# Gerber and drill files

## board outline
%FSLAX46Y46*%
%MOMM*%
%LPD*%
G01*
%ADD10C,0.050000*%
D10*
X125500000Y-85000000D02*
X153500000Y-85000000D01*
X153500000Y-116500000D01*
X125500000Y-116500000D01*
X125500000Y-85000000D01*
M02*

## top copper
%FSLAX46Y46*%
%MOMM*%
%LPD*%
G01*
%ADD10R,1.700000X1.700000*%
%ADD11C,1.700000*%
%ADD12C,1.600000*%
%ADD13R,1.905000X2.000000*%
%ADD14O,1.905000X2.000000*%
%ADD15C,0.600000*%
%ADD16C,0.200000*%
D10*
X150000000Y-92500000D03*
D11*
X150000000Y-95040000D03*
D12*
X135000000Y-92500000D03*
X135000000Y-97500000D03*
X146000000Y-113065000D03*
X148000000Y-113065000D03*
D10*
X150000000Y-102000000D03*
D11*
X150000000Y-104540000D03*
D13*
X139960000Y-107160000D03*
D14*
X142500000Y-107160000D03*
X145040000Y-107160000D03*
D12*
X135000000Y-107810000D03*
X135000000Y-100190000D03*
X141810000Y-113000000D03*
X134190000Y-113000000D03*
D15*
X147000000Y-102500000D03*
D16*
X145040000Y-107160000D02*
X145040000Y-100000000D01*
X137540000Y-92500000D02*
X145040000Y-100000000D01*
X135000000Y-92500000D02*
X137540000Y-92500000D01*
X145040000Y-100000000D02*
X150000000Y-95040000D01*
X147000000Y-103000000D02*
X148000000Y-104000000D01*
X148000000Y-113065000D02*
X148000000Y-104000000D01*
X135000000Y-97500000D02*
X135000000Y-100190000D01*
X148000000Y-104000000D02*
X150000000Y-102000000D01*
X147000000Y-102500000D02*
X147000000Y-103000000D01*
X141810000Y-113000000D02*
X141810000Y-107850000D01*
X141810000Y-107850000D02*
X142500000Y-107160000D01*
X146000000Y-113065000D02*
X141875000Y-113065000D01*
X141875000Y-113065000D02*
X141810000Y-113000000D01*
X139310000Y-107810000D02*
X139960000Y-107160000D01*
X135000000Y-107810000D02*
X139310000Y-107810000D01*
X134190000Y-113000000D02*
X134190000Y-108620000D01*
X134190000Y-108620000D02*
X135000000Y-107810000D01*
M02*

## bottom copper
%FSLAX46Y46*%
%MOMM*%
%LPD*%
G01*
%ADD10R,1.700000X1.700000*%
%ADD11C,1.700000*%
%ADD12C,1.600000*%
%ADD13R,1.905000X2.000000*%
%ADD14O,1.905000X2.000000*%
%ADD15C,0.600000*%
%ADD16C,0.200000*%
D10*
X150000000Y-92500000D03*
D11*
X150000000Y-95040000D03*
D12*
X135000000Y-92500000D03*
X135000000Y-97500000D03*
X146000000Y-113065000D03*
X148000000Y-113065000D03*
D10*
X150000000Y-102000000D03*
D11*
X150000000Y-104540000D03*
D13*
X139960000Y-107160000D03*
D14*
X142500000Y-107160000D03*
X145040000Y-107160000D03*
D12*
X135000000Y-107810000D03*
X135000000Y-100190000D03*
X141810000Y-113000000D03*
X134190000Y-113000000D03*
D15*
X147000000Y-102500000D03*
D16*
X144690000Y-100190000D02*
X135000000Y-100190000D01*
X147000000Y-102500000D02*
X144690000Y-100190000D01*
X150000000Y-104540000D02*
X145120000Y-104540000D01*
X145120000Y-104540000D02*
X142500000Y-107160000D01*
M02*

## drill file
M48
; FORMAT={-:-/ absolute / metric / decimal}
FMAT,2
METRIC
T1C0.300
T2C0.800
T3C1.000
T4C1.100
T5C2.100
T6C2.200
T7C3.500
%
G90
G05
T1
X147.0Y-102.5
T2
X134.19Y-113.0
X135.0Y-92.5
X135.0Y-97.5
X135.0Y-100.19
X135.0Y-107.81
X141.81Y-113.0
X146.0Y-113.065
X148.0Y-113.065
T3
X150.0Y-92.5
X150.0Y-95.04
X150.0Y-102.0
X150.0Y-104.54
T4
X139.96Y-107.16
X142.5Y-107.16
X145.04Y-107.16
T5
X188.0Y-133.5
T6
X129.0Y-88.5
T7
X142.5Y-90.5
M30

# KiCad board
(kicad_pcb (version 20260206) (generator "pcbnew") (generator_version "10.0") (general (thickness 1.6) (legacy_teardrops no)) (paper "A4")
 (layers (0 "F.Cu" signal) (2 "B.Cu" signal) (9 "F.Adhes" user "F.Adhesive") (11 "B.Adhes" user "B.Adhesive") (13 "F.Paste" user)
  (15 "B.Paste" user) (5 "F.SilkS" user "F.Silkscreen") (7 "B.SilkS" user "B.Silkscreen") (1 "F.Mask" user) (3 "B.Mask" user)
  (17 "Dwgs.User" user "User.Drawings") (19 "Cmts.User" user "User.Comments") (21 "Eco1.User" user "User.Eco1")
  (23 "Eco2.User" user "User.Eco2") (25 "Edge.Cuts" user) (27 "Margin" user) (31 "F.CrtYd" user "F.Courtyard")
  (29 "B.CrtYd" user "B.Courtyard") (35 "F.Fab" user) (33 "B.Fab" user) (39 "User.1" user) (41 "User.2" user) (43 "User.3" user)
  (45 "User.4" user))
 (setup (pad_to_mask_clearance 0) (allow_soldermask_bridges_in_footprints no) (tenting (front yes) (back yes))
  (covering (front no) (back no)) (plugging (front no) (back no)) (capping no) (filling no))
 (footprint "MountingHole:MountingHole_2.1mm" (layer "F.Cu") (at 188 133.5)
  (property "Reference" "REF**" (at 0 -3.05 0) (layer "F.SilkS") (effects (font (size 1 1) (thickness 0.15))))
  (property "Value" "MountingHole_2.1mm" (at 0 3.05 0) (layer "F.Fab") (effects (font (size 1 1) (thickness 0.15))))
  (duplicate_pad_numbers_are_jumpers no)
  (pad "" np_thru_hole circle (at 0 0) (size 2.1 2.1) (drill 2.1) (layers "*.Cu" "*.Mask")))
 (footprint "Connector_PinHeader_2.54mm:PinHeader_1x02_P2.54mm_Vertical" (layer "F.Cu") (at 150 92.5)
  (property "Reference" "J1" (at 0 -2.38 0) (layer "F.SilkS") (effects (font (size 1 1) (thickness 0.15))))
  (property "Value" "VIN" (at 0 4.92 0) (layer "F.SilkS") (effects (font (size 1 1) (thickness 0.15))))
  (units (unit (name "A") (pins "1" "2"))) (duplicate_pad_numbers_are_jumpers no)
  (pad "1" thru_hole rect (at 0 0) (size 1.7 1.7) (drill 1) (layers "*.Cu" "*.Mask") (remove_unused_layers no) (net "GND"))
  (pad "2" thru_hole circle (at 0 2.54) (size 1.7 1.7) (drill 1) (layers "*.Cu" "*.Mask") (remove_unused_layers no) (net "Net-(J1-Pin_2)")))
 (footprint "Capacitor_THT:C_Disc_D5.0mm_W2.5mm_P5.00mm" (layer "F.Cu") (at 135 92.5 -90)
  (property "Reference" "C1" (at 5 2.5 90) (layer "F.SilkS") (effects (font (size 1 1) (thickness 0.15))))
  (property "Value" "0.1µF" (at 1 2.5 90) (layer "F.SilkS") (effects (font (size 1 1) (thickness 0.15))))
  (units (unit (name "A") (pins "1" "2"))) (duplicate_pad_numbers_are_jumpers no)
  (pad "1" thru_hole circle (at 0 0 270) (size 1.6 1.6) (drill 0.8) (layers "*.Cu" "*.Mask") (remove_unused_layers no)
   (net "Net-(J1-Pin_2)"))
  (pad "2" thru_hole circle (at 5 0 270) (size 1.6 1.6) (drill 0.8) (layers "*.Cu" "*.Mask") (remove_unused_layers no) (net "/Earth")))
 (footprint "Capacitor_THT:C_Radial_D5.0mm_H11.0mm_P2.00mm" (layer "F.Cu") (at 146 113.065)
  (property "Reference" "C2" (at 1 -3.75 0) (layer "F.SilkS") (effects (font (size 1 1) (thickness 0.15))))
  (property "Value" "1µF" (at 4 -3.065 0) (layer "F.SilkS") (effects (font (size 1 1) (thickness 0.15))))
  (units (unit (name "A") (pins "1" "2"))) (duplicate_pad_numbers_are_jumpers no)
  (pad "1" thru_hole circle (at 0 0) (size 1.6 1.6) (drill 0.8) (layers "*.Cu" "*.Mask") (remove_unused_layers no) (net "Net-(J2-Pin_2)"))
  (pad "2" thru_hole circle (at 2 0) (size 1.6 1.6) (drill 0.8) (layers "*.Cu" "*.Mask") (remove_unused_layers no) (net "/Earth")))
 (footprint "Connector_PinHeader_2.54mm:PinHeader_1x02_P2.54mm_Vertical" (layer "F.Cu") (at 150 102)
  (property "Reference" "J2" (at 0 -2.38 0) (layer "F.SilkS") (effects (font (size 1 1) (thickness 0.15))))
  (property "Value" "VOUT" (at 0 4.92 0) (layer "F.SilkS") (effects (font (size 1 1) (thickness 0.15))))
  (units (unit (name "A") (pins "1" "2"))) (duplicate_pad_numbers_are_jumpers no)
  (pad "1" thru_hole rect (at 0 0) (size 1.7 1.7) (drill 1) (layers "*.Cu" "*.Mask") (remove_unused_layers no) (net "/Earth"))
  (pad "2" thru_hole circle (at 0 2.54) (size 1.7 1.7) (drill 1) (layers "*.Cu" "*.Mask") (remove_unused_layers no) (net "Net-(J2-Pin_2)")))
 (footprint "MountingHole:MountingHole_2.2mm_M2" (layer "F.Cu") (at 129 88.5)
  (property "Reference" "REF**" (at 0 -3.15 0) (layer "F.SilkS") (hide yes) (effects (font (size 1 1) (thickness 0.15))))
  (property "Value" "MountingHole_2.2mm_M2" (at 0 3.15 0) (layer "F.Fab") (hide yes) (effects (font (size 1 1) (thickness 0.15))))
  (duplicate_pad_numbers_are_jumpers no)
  (pad "" np_thru_hole circle (at 0 0) (size 2.2 2.2) (drill 2.2) (layers "*.Cu" "*.Mask")))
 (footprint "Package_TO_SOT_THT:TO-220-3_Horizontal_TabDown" (layer "F.Cu") (at 139.96 107.16)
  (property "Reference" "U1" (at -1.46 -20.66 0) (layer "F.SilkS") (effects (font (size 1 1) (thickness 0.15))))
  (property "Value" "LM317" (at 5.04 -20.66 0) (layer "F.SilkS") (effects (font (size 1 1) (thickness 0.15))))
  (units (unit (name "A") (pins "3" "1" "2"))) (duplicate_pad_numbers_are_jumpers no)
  (pad "" np_thru_hole circle (at 2.54 -16.66) (size 3.5 3.5) (drill 3.5) (layers "*.Cu" "*.Mask"))
  (pad "1" thru_hole rect (at 0 0) (size 1.905 2) (drill 1.1) (layers "*.Cu" "*.Mask") (remove_unused_layers no) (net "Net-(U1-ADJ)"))
  (pad "2" thru_hole oval (at 2.54 0) (size 1.905 2) (drill 1.1) (layers "*.Cu" "*.Mask") (remove_unused_layers no) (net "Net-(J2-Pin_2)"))
  (pad "3" thru_hole oval (at 5.08 0) (size 1.905 2) (drill 1.1) (layers "*.Cu" "*.Mask") (remove_unused_layers no) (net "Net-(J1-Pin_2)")))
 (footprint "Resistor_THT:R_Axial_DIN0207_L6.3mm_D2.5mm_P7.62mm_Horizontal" (layer "F.Cu") (at 135 107.81 90)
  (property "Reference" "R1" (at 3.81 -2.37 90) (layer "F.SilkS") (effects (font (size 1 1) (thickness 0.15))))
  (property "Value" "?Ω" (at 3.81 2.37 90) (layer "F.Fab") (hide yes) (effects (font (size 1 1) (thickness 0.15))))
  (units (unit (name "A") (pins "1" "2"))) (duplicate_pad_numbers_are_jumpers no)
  (pad "1" thru_hole circle (at 0 0 90) (size 1.6 1.6) (drill 0.8) (layers "*.Cu" "*.Mask") (remove_unused_layers no) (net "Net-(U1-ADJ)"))
  (pad "2" thru_hole circle (at 7.62 0 90) (size 1.6 1.6) (drill 0.8) (layers "*.Cu" "*.Mask") (remove_unused_layers no) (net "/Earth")))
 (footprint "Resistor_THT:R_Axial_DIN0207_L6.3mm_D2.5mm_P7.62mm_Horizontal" (layer "F.Cu") (at 141.81 113 180)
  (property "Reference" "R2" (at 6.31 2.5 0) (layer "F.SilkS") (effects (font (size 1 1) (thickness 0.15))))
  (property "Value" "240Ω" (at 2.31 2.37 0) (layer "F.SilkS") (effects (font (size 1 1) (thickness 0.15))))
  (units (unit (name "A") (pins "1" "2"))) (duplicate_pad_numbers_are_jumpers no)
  (pad "1" thru_hole circle (at 0 0 180) (size 1.6 1.6) (drill 0.8) (layers "*.Cu" "*.Mask") (remove_unused_layers no)
   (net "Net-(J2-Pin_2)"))
  (pad "2" thru_hole circle (at 7.62 0 180) (size 1.6 1.6) (drill 0.8) (layers "*.Cu" "*.Mask") (remove_unused_layers no)
   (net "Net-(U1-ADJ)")))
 (gr_rect (start 125.5 85) (end 153.5 116.5) (stroke (width 0.05) (type default)) (fill no) (layer "Edge.Cuts"))
 (segment (start 145.04 107.16) (end 145.04 100) (width 0.2) (layer "F.Cu") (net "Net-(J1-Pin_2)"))
 (segment (start 137.54 92.5) (end 145.04 100) (width 0.2) (layer "F.Cu") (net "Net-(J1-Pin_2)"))
 (segment (start 135 92.5) (end 137.54 92.5) (width 0.2) (layer "F.Cu") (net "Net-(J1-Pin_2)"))
 (segment (start 145.04 100) (end 150 95.04) (width 0.2) (layer "F.Cu") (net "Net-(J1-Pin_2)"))
 (segment (start 147 103) (end 148 104) (width 0.2) (layer "F.Cu") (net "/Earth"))
 (segment (start 148 113.065) (end 148 104) (width 0.2) (layer "F.Cu") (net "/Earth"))
 (segment (start 135 97.5) (end 135 100.19) (width 0.2) (layer "F.Cu") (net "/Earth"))
 (segment (start 148 104) (end 150 102) (width 0.2) (layer "F.Cu") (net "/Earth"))
 (segment (start 147 102.5) (end 147 103) (width 0.2) (layer "F.Cu") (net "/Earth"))
 (via (at 147 102.5) (size 0.6) (drill 0.3) (layers "F.Cu" "B.Cu") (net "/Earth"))
 (segment (start 144.69 100.19) (end 135 100.19) (width 0.2) (layer "B.Cu") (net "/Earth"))
 (segment (start 147 102.5) (end 144.69 100.19) (width 0.2) (layer "B.Cu") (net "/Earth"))
 (segment (start 141.81 113) (end 141.81 107.85) (width 0.2) (layer "F.Cu") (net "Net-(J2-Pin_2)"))
 (segment (start 141.81 107.85) (end 142.5 107.16) (width 0.2) (layer "F.Cu") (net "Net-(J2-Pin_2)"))
 (segment (start 146 113.065) (end 141.875 113.065) (width 0.2) (layer "F.Cu") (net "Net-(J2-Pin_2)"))
 (segment (start 141.875 113.065) (end 141.81 113) (width 0.2) (layer "F.Cu") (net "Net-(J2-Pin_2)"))
 (segment (start 150 104.54) (end 145.12 104.54) (width 0.2) (layer "B.Cu") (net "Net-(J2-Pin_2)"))
 (segment (start 145.12 104.54) (end 142.5 107.16) (width 0.2) (layer "B.Cu") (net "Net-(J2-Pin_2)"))
 (segment (start 139.31 107.81) (end 139.96 107.16) (width 0.2) (layer "F.Cu") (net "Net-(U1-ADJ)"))
 (segment (start 135 107.81) (end 139.31 107.81) (width 0.2) (layer "F.Cu") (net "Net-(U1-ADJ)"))
 (segment (start 134.19 113) (end 134.19 108.62) (width 0.2) (layer "F.Cu") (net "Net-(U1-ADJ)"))
 (segment (start 134.19 108.62) (end 135 107.81) (width 0.2) (layer "F.Cu") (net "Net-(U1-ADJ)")))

